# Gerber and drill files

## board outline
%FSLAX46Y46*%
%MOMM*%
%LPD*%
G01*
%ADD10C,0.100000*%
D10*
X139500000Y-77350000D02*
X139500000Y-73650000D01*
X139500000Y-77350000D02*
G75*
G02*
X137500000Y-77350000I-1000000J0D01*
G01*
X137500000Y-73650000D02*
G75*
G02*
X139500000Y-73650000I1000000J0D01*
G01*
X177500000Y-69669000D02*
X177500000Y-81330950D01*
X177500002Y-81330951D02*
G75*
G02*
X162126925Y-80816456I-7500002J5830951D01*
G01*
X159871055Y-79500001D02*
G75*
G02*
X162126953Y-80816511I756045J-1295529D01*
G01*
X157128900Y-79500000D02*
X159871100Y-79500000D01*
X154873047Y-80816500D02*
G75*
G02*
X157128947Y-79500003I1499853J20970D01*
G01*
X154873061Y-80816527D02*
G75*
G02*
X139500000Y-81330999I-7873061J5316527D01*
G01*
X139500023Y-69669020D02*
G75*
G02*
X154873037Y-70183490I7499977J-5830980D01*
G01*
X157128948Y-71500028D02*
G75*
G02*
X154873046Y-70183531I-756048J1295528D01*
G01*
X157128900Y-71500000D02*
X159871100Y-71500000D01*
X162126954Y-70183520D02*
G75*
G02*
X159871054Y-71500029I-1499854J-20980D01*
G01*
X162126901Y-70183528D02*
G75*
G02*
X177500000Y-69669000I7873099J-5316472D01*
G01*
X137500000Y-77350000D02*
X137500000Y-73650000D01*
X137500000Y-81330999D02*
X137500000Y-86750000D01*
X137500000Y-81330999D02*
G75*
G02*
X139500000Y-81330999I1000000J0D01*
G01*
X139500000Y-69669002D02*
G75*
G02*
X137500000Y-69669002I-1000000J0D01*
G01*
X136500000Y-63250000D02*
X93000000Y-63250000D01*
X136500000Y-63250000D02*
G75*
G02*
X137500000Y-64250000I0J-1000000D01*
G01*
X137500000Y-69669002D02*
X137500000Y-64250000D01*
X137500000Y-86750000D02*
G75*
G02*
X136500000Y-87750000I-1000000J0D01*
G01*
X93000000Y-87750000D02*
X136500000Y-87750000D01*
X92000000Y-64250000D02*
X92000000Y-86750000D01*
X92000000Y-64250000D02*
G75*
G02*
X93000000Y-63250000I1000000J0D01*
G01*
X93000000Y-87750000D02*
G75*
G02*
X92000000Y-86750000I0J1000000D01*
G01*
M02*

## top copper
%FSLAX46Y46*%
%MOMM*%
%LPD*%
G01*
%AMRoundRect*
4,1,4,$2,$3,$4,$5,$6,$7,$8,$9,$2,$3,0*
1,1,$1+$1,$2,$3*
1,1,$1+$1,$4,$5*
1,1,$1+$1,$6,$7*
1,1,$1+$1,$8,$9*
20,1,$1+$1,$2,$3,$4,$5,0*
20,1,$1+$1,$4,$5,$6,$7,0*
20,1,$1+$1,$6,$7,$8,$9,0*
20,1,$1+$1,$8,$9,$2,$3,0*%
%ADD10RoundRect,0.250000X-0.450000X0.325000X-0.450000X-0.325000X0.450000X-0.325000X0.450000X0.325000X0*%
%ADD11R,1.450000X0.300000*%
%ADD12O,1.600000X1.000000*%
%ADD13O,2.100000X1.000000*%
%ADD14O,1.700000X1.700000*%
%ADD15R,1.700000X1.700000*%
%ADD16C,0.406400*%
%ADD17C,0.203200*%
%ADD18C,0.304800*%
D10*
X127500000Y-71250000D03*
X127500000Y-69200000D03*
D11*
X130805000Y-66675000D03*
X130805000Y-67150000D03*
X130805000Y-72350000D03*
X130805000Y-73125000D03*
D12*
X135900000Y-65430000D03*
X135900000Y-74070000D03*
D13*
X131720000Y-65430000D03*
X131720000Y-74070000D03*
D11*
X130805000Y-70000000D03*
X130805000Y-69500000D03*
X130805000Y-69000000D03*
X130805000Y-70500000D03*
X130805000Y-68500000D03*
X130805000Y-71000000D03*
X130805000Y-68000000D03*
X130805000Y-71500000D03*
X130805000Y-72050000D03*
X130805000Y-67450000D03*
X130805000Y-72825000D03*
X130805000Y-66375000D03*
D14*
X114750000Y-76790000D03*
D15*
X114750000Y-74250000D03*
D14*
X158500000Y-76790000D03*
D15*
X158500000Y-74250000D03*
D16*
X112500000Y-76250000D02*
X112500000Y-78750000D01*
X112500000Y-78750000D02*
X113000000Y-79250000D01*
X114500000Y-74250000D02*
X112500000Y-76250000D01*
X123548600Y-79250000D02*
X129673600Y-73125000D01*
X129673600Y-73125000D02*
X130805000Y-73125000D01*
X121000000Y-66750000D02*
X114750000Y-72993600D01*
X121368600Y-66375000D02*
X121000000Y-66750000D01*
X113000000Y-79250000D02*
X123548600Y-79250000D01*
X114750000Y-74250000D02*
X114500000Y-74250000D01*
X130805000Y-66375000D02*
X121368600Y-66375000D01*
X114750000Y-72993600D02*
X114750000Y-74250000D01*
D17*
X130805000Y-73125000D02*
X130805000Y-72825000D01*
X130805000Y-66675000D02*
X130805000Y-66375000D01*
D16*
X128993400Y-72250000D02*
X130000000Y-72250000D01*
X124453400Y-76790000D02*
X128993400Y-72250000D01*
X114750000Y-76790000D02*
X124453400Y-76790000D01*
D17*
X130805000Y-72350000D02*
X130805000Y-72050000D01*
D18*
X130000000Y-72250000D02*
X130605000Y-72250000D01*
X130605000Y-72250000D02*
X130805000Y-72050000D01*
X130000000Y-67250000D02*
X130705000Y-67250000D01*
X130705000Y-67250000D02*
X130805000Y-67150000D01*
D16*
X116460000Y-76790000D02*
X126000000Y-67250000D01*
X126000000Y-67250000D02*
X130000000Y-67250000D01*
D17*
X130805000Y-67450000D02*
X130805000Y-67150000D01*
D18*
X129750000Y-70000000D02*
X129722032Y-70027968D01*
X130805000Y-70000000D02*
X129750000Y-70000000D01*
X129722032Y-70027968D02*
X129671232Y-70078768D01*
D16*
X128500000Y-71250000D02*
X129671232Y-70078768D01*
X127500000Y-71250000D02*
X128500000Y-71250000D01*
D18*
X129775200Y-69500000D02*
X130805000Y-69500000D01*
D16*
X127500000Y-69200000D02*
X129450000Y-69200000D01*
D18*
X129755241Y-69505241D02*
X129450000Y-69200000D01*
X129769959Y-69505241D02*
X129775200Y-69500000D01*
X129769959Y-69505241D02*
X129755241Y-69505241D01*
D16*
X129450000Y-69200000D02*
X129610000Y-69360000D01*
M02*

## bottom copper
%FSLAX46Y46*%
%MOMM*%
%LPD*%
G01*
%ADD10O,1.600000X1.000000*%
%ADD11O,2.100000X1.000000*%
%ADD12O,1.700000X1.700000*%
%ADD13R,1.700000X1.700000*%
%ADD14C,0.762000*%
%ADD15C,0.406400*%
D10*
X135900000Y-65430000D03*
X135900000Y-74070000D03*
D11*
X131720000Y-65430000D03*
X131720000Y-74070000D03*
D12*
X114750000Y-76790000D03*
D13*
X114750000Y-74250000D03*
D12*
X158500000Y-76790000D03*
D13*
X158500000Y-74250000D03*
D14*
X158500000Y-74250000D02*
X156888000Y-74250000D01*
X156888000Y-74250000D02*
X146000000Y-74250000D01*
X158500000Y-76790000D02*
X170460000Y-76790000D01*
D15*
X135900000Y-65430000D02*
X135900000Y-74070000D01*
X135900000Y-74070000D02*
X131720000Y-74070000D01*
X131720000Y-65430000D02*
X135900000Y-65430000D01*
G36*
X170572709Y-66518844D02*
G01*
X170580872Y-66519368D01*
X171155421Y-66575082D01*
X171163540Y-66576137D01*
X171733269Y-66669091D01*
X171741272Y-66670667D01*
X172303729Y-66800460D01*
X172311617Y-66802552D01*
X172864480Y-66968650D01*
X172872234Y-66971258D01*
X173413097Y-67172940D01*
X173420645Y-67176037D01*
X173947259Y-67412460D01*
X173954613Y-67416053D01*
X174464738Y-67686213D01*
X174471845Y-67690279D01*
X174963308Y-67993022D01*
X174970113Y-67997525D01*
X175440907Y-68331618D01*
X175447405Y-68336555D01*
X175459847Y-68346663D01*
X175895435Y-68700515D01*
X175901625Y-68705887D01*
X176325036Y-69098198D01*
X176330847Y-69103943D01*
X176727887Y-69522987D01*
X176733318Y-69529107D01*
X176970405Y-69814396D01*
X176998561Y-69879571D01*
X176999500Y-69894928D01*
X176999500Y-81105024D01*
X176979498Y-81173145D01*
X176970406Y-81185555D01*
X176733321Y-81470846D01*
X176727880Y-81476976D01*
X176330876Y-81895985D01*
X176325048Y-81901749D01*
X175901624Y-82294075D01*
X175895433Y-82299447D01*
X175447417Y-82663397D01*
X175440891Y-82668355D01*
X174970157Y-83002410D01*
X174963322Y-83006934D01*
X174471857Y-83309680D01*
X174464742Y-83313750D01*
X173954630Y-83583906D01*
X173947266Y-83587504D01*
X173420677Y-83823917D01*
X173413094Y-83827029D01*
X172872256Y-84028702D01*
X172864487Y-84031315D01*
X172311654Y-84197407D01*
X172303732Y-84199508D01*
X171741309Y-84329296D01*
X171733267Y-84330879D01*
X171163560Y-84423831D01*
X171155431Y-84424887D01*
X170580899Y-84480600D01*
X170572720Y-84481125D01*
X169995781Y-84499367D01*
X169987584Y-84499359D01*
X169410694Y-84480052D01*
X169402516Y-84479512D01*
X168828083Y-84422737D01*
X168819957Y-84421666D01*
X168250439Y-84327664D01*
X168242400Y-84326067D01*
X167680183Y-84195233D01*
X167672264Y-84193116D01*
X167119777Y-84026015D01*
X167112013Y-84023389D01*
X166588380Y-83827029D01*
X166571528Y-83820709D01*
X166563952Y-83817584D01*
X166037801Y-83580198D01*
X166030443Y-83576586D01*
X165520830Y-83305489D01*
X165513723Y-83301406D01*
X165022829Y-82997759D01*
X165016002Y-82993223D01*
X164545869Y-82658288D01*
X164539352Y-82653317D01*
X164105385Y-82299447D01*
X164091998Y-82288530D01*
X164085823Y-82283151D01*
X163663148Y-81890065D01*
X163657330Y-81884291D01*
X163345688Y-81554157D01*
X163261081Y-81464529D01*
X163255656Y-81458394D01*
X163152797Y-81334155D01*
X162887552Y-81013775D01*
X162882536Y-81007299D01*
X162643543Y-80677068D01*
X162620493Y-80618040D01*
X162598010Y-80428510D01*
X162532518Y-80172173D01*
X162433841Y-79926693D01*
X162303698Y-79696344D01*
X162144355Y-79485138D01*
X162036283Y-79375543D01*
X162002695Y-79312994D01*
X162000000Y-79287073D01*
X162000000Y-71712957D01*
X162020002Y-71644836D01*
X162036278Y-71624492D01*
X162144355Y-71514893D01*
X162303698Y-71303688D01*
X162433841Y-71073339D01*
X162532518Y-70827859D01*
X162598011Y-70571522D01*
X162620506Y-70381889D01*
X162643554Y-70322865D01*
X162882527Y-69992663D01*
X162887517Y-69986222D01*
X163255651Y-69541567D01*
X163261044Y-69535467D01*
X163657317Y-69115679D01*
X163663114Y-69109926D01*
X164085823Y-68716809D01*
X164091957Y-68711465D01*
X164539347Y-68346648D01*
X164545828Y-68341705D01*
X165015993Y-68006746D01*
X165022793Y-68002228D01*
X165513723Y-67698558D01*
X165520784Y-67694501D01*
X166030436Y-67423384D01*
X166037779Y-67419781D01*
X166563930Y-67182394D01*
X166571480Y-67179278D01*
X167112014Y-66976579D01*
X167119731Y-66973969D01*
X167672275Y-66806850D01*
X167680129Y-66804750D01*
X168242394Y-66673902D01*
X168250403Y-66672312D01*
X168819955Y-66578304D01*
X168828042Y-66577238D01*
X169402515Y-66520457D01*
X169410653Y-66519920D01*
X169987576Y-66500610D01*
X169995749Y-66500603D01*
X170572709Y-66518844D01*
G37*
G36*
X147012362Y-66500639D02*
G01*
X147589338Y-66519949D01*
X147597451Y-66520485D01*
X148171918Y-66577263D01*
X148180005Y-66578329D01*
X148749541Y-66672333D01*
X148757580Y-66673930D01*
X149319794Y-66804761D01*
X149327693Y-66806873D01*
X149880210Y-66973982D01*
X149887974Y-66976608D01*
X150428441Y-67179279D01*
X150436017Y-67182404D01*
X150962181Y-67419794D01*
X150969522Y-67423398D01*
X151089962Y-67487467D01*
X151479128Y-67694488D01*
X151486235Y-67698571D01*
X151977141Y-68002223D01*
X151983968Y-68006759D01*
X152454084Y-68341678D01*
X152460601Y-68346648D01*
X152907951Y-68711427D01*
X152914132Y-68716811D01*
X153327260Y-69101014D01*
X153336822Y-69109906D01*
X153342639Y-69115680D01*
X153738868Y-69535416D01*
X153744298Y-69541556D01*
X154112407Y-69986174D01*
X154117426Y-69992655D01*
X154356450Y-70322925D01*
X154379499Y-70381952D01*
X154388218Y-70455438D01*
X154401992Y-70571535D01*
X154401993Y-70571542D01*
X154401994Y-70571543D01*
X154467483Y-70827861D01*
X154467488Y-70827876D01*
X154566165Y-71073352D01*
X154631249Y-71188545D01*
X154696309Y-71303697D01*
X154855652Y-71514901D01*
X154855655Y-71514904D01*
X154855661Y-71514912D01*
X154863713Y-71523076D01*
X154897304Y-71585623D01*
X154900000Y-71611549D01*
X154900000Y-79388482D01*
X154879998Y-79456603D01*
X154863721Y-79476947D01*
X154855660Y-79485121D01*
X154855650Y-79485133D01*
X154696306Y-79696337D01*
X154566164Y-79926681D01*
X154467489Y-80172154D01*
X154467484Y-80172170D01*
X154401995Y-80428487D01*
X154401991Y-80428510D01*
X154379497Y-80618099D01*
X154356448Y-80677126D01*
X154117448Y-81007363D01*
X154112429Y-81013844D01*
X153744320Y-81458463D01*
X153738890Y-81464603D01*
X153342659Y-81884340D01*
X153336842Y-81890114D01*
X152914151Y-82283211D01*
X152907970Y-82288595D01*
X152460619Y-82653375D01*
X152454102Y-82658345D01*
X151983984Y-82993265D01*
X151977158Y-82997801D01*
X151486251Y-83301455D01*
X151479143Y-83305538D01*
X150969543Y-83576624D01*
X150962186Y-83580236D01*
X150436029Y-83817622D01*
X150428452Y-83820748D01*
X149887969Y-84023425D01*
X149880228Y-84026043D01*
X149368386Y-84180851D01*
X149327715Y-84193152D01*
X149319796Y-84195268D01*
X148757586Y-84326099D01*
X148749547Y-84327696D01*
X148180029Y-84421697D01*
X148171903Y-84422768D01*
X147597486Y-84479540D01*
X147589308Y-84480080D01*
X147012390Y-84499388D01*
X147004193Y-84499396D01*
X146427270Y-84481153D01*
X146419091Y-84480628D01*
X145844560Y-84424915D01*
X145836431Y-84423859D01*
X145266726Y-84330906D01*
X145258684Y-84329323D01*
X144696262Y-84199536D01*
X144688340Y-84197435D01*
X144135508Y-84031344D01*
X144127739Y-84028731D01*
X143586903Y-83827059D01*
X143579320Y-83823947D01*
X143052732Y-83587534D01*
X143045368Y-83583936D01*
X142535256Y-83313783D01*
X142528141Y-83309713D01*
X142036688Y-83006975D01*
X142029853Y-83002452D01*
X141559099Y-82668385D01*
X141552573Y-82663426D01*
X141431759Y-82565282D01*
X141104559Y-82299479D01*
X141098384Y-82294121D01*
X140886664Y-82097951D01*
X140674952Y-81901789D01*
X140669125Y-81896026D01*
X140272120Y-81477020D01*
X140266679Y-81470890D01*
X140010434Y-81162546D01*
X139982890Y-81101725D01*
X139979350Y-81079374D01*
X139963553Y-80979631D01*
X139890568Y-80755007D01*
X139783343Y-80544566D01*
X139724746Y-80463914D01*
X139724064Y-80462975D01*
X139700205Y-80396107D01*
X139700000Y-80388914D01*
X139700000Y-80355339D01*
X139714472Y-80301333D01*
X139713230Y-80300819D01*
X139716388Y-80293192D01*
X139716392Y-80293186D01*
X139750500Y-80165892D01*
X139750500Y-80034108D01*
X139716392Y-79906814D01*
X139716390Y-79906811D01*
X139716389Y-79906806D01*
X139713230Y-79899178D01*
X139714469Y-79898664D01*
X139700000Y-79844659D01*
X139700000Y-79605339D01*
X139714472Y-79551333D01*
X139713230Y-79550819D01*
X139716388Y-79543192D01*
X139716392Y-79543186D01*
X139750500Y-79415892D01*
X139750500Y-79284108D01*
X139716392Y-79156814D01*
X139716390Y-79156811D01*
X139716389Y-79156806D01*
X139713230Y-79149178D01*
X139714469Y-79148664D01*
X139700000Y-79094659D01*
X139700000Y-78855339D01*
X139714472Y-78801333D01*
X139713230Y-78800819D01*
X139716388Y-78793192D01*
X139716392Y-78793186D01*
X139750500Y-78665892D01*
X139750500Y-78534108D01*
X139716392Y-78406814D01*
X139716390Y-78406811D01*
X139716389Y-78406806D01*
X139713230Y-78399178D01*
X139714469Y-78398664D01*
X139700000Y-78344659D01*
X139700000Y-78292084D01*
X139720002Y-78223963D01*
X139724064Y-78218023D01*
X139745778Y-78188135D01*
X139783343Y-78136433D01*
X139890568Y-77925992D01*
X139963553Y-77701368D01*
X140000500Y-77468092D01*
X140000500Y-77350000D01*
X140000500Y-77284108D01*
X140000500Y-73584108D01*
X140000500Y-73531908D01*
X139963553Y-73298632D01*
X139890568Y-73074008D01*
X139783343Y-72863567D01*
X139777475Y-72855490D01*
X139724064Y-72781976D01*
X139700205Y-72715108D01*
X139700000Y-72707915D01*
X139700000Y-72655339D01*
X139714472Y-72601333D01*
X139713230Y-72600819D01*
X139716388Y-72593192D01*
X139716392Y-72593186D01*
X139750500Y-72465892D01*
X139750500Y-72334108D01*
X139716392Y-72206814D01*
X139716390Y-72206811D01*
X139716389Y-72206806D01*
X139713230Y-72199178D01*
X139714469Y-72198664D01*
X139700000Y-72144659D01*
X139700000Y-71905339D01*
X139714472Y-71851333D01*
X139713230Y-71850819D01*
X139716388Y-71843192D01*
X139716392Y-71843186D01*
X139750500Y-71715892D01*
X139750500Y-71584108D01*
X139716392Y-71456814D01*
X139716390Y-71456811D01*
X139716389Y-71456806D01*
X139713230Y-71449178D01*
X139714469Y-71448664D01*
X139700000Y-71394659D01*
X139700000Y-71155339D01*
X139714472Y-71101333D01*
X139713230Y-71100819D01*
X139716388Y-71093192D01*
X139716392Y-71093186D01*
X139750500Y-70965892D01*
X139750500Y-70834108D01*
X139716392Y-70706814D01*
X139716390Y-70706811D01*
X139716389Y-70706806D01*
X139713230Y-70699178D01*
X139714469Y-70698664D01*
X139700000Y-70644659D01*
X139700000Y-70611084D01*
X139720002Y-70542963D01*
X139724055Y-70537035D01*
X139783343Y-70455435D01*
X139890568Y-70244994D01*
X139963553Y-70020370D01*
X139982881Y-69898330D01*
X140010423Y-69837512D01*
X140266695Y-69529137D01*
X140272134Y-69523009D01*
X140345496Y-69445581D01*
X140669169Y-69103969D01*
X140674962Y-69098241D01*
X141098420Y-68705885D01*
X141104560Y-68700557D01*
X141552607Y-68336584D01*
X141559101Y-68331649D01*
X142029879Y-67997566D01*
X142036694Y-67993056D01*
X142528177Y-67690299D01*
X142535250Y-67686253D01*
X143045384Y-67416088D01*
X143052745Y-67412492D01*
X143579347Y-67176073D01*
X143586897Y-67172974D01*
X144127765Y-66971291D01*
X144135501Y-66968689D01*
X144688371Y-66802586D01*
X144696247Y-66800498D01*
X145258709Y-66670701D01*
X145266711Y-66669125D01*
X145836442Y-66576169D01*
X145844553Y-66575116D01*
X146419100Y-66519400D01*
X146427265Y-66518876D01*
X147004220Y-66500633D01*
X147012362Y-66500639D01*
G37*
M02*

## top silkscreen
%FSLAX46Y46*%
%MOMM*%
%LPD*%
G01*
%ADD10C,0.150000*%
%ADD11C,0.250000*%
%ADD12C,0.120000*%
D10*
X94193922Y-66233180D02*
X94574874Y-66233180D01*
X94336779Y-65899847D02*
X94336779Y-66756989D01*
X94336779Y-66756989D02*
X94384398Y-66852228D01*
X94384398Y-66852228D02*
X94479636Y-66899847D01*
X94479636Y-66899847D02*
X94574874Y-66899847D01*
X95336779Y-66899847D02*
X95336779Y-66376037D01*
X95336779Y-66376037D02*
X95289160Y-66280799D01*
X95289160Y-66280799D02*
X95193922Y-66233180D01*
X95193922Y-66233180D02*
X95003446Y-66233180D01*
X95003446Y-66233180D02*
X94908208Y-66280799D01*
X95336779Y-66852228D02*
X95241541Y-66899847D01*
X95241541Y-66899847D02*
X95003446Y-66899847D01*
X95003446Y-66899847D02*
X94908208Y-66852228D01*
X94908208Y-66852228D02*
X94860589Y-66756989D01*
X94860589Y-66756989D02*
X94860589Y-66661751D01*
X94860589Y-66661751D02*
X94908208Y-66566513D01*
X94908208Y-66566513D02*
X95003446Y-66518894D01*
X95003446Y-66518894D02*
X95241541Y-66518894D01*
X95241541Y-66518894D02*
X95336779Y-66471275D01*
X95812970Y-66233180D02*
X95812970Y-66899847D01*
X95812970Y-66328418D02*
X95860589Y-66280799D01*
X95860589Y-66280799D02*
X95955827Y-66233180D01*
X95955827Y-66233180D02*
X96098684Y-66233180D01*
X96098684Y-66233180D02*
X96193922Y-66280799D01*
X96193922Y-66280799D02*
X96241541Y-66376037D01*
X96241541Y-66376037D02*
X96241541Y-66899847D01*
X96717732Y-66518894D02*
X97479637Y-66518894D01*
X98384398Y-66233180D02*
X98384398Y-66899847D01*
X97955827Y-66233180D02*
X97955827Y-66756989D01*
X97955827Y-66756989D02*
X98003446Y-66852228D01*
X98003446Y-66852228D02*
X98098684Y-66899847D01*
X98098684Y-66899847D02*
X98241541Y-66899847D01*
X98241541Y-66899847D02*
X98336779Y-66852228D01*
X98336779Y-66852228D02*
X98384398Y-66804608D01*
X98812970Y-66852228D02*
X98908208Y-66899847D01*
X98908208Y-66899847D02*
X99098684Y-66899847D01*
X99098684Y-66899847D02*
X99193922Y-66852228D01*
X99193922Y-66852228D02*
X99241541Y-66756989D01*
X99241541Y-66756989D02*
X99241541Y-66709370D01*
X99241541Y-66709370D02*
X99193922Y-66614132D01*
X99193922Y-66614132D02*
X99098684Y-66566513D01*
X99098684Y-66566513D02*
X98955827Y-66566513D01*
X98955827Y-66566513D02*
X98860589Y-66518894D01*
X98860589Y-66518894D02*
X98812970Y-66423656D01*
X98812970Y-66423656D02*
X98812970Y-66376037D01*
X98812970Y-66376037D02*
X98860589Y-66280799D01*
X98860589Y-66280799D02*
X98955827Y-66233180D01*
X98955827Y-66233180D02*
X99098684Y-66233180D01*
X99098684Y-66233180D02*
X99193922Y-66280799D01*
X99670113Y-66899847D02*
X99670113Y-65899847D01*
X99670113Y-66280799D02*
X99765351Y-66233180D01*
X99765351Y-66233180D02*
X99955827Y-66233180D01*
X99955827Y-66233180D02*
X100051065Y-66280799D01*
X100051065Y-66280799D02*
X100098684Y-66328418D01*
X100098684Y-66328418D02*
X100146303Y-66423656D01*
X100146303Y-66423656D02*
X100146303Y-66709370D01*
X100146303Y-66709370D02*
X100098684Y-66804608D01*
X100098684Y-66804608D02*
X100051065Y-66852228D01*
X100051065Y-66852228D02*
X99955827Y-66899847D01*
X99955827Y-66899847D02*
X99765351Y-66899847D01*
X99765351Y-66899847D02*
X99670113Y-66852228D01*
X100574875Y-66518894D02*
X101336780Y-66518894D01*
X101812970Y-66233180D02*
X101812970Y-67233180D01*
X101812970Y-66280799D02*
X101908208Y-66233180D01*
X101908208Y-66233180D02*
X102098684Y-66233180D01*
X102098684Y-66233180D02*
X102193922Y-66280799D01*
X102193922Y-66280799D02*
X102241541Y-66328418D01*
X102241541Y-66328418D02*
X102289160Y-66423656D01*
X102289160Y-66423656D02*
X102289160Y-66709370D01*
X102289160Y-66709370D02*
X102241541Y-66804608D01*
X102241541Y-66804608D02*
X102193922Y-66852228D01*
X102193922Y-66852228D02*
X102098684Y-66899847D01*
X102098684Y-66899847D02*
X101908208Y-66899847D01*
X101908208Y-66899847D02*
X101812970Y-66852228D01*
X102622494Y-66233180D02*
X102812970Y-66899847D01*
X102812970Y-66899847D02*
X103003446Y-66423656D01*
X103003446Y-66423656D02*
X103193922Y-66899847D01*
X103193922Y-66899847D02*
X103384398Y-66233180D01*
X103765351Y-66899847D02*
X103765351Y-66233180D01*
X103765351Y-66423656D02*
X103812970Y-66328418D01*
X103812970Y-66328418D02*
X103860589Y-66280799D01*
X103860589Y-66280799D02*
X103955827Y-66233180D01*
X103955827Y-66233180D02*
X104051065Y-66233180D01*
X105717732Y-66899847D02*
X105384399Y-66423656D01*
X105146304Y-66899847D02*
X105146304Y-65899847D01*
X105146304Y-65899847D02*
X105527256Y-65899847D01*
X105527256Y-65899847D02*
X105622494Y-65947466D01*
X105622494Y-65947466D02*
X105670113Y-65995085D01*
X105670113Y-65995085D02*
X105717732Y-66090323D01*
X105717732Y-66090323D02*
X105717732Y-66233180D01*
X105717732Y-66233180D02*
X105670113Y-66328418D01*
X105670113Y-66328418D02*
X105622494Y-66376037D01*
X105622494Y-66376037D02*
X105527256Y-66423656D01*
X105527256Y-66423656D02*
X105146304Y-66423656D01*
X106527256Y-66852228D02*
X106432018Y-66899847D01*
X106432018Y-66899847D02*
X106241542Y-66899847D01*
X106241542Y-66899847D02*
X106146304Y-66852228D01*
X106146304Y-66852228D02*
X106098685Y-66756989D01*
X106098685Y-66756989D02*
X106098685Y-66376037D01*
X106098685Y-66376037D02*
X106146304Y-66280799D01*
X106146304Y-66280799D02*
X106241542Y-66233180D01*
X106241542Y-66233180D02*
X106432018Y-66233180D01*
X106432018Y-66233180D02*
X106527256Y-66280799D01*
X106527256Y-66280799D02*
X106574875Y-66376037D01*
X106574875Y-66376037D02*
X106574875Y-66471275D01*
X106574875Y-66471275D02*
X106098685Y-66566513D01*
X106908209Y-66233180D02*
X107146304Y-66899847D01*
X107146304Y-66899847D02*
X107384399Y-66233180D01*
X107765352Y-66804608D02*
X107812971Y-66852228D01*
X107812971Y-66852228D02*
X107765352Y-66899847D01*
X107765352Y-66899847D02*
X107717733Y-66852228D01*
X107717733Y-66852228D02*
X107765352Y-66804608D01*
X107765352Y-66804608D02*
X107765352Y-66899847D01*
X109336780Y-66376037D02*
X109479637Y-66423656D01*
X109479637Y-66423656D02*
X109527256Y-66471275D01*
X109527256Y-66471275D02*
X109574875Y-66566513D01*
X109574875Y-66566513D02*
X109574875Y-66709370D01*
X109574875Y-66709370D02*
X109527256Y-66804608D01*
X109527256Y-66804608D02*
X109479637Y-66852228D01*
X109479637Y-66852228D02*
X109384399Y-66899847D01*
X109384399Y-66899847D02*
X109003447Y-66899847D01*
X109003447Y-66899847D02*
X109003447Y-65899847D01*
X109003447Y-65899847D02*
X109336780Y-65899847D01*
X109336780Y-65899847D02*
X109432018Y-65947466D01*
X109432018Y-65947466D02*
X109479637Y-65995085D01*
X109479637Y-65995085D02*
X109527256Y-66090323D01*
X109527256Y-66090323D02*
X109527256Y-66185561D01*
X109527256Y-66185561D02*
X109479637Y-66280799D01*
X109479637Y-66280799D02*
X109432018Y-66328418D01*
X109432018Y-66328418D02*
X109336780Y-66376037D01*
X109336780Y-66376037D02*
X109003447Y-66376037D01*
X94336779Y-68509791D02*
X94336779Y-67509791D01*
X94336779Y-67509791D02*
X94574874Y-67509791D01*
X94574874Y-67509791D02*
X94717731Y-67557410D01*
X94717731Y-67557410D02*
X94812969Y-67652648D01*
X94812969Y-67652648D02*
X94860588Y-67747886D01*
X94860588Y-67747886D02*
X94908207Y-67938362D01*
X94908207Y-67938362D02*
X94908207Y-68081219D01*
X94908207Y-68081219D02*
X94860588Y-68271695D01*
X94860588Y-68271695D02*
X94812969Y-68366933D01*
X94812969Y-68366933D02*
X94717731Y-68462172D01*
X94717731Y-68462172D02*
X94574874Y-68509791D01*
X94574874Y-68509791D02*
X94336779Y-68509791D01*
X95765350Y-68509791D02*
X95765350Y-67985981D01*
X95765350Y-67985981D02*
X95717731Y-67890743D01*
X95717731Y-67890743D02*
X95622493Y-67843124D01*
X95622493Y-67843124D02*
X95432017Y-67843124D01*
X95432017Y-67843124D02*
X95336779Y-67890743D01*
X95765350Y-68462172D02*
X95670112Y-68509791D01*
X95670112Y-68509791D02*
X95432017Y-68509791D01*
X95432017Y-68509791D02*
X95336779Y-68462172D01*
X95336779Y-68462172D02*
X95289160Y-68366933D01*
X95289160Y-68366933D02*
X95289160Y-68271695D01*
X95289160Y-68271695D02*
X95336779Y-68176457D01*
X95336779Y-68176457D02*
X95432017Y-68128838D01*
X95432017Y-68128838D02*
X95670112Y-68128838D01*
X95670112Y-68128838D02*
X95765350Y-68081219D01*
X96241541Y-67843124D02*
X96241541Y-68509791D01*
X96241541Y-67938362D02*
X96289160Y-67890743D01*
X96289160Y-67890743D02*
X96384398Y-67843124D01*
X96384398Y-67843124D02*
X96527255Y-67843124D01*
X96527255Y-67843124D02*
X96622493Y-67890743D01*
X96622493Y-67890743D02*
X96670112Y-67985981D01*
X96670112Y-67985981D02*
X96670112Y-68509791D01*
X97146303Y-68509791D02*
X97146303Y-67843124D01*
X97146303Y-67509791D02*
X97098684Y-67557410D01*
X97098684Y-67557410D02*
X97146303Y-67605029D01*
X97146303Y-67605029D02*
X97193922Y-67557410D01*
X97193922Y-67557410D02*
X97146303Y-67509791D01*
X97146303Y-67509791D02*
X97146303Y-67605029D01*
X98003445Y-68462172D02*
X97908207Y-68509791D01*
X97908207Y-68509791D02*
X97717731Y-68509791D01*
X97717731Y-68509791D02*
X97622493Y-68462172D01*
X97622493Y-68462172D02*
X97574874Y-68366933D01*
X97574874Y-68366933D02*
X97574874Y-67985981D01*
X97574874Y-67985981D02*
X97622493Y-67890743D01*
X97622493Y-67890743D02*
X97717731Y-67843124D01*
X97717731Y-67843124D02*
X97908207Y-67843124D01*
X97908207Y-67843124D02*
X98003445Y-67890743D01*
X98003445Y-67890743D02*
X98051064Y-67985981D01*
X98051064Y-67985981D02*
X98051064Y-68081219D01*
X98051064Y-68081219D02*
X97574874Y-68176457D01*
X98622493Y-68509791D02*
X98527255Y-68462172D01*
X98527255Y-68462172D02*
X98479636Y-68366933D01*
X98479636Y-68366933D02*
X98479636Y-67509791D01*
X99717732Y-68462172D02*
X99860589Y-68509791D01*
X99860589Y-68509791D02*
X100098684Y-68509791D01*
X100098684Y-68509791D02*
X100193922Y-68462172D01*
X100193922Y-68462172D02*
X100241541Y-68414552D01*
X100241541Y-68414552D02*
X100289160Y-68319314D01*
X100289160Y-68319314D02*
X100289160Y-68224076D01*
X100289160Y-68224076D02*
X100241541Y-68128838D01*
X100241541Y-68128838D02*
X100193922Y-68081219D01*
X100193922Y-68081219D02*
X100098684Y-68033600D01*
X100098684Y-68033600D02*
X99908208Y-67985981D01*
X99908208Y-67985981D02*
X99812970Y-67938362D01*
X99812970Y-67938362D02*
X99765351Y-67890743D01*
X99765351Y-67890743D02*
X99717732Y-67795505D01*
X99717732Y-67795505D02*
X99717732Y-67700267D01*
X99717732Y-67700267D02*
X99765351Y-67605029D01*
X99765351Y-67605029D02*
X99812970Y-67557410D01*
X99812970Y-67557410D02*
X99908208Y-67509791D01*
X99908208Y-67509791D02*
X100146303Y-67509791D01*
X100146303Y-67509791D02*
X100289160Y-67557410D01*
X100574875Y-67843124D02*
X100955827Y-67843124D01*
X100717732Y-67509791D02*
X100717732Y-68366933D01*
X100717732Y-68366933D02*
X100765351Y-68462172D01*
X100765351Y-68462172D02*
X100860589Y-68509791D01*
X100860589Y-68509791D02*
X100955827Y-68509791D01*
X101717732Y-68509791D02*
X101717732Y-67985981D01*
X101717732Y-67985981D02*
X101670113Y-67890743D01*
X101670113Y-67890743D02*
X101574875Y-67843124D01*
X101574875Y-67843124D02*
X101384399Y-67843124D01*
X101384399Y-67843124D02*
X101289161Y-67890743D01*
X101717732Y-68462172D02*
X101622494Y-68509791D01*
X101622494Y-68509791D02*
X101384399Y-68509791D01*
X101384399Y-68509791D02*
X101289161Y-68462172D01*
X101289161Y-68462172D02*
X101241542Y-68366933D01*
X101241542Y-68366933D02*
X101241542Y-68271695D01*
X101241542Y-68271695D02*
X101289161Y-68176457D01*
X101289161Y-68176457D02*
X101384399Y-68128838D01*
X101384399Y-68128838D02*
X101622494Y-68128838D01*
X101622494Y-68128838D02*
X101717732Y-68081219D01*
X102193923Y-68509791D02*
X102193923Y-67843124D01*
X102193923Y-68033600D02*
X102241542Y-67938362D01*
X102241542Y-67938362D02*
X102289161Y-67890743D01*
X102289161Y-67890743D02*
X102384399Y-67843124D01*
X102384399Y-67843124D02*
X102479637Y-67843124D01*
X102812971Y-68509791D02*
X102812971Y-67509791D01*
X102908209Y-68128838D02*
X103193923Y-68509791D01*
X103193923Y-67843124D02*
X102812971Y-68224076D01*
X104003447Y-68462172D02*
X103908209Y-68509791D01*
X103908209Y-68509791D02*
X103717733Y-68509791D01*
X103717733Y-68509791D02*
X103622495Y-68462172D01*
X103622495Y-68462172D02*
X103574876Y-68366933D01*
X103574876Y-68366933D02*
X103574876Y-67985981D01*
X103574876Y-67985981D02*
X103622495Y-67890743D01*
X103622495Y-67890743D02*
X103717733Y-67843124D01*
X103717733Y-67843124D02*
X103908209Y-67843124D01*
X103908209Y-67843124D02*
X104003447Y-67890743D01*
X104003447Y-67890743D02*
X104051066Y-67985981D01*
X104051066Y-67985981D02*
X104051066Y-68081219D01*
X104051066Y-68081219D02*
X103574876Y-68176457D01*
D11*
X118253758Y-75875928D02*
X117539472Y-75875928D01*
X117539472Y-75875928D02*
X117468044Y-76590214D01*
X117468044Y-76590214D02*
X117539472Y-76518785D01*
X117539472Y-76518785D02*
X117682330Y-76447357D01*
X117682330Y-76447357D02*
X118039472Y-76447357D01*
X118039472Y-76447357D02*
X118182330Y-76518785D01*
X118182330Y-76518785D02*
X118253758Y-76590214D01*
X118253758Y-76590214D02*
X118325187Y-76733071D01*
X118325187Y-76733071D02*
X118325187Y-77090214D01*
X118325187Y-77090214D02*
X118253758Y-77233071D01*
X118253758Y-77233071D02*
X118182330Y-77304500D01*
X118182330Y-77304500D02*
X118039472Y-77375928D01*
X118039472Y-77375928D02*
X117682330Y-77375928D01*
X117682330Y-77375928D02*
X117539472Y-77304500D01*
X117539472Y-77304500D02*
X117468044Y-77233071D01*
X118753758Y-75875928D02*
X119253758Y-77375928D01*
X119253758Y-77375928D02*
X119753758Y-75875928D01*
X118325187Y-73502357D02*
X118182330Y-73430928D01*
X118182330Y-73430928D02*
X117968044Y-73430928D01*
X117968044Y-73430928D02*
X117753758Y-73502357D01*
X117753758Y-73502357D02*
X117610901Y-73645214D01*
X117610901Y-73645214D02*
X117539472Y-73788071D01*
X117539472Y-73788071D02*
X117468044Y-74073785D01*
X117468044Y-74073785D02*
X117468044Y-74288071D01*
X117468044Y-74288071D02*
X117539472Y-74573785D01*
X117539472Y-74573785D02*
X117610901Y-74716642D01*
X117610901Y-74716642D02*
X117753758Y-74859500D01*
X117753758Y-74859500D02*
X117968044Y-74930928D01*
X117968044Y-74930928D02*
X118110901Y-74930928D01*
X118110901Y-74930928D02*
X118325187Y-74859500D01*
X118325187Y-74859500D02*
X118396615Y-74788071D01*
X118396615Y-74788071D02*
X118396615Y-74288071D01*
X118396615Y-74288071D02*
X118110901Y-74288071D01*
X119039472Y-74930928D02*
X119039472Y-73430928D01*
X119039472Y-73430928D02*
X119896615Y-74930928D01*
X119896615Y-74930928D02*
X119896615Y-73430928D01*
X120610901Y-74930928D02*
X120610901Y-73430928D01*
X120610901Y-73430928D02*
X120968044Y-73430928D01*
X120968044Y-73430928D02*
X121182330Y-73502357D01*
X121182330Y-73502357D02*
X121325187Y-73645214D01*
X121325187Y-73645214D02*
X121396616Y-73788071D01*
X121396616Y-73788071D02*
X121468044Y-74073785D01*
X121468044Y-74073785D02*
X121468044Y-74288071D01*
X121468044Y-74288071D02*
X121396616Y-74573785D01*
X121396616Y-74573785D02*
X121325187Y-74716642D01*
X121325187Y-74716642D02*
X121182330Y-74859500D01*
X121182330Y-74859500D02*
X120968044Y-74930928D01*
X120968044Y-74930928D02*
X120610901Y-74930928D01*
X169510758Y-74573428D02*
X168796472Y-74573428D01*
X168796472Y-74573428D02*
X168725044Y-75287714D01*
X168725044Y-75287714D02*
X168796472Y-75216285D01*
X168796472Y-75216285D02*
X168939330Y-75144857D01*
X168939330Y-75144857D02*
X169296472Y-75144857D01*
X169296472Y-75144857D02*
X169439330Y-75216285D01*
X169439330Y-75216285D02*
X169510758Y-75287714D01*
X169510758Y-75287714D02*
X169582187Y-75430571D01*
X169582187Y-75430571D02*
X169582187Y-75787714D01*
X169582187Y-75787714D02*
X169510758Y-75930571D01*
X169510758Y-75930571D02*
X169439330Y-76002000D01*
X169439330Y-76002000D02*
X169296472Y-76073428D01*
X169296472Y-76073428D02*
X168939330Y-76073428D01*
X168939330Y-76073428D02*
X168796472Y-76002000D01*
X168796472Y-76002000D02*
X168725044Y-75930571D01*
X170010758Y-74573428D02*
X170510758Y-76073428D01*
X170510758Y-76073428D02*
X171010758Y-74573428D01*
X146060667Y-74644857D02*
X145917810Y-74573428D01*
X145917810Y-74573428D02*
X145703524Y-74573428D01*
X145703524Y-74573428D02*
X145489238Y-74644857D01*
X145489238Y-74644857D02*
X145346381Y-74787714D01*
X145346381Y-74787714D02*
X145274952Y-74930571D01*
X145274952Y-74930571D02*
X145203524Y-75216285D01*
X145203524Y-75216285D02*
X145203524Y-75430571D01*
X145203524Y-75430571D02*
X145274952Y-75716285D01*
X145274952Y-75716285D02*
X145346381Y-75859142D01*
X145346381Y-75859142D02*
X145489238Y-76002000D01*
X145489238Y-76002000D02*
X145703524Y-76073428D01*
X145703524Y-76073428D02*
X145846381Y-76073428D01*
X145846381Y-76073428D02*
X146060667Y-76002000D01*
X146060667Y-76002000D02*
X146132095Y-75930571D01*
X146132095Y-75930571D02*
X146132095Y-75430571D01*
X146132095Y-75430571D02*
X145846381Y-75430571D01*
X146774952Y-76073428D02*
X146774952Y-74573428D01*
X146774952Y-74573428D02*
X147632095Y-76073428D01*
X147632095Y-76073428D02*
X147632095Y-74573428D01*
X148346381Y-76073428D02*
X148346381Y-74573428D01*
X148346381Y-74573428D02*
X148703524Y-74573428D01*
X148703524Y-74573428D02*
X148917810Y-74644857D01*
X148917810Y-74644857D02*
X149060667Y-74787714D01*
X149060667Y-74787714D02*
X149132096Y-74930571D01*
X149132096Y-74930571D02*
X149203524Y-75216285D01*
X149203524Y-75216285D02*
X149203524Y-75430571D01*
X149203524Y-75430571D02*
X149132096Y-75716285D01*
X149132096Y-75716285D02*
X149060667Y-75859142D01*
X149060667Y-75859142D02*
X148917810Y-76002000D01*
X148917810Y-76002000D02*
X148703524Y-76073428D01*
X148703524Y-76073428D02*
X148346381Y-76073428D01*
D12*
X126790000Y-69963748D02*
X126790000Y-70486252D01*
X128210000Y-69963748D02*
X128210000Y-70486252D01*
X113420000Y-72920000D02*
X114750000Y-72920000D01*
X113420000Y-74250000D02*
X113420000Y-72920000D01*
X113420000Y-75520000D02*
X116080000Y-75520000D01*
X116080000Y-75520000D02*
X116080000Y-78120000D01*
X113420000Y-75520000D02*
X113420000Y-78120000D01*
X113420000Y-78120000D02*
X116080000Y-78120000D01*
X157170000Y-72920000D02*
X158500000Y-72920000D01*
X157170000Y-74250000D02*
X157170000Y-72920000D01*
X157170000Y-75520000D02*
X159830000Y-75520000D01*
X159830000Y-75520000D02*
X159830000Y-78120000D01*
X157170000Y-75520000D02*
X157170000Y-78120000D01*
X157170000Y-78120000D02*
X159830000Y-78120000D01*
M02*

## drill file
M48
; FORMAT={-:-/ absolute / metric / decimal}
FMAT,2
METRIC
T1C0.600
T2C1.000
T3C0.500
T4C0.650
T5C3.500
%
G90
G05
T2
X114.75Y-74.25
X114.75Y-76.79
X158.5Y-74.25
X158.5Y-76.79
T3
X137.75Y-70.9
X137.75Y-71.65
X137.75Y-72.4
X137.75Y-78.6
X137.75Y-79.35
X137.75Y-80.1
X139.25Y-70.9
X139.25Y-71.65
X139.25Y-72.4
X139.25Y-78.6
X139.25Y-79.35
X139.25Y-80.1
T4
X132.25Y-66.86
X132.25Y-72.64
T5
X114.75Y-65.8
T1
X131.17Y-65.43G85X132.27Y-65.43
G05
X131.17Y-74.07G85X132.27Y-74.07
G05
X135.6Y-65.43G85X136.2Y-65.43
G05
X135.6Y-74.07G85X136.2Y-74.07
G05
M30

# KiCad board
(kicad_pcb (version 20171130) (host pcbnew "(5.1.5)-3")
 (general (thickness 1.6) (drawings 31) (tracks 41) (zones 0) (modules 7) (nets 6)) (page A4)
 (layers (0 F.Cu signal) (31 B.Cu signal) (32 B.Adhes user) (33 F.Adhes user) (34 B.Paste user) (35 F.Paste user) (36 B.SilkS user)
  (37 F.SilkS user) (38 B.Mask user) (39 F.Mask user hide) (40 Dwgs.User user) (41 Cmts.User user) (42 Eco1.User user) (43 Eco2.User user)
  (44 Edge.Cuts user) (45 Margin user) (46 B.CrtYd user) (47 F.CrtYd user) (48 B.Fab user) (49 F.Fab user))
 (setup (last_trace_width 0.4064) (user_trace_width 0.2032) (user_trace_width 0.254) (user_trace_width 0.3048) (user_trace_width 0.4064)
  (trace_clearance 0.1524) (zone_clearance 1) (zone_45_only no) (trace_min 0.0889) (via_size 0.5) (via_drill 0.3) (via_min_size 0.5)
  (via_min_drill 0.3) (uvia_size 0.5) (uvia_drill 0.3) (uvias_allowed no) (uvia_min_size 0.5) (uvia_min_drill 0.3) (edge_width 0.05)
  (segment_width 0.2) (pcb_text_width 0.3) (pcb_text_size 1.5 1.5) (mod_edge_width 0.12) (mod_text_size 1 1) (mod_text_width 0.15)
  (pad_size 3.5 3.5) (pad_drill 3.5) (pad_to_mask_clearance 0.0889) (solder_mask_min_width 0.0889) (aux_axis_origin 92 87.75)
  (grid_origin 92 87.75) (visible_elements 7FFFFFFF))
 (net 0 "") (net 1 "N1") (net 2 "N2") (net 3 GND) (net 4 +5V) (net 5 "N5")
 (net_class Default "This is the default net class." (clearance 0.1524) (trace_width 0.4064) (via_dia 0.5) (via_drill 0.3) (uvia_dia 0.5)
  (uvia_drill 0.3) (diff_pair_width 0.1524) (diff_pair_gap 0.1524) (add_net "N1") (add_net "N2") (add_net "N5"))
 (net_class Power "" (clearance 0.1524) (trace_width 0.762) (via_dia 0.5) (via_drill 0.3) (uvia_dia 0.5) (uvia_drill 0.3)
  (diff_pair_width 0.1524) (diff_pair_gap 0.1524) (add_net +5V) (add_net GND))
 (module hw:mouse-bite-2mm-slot (layer F.Cu) (at 138.5 79.35 90)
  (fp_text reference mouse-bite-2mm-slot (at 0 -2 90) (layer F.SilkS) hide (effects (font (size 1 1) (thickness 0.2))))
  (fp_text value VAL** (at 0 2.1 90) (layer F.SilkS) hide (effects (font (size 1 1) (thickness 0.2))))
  (pad "" np_thru_hole circle (at 0 -0.75 90) (size 0.5 0.5) (drill 0.5) (layers *.Cu *.Mask))
  (pad "" np_thru_hole circle (at 0 0.75 90) (size 0.5 0.5) (drill 0.5) (layers *.Cu *.Mask))
  (pad "" np_thru_hole circle (at 0.75 -0.75 90) (size 0.5 0.5) (drill 0.5) (layers *.Cu *.Mask))
  (pad "" np_thru_hole circle (at -0.75 -0.75 90) (size 0.5 0.5) (drill 0.5) (layers *.Cu *.Mask))
  (pad "" np_thru_hole circle (at -0.75 0.75 90) (size 0.5 0.5) (drill 0.5) (layers *.Cu *.Mask))
  (pad "" np_thru_hole circle (at 0.75 0.75 90) (size 0.5 0.5) (drill 0.5) (layers *.Cu *.Mask)))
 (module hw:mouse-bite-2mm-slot (layer F.Cu) (at 138.5 71.65 90)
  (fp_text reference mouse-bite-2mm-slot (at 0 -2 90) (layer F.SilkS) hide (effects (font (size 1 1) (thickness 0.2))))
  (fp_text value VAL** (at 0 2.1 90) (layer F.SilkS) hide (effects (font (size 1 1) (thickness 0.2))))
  (pad "" np_thru_hole circle (at 0 -0.75 90) (size 0.5 0.5) (drill 0.5) (layers *.Cu *.Mask))
  (pad "" np_thru_hole circle (at 0 0.75 90) (size 0.5 0.5) (drill 0.5) (layers *.Cu *.Mask))
  (pad "" np_thru_hole circle (at 0.75 -0.75 90) (size 0.5 0.5) (drill 0.5) (layers *.Cu *.Mask))
  (pad "" np_thru_hole circle (at -0.75 -0.75 90) (size 0.5 0.5) (drill 0.5) (layers *.Cu *.Mask))
  (pad "" np_thru_hole circle (at -0.75 0.75 90) (size 0.5 0.5) (drill 0.5) (layers *.Cu *.Mask))
  (pad "" np_thru_hole circle (at 0.75 0.75 90) (size 0.5 0.5) (drill 0.5) (layers *.Cu *.Mask)))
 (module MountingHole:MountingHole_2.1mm (layer F.Cu) (at 114.75 65.8)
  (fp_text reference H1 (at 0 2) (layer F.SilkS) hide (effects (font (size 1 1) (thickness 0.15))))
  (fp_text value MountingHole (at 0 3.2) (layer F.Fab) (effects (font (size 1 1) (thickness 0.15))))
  (pad "" np_thru_hole circle (at 0 0) (size 3.5 3.5) (drill 3.5) (layers *.Cu *.Mask)))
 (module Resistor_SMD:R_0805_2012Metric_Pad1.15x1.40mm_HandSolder (layer F.Cu) (at 127.5 70.225 270)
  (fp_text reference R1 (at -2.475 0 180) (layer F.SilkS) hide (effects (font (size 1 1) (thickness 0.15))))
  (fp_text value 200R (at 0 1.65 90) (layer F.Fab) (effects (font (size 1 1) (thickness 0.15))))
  (fp_line (start -0.261252 0.71) (end 0.261252 0.71) (layer F.SilkS) (width 0.12))
  (fp_line (start -0.261252 -0.71) (end 0.261252 -0.71) (layer F.SilkS) (width 0.12))
  (pad 2 smd roundrect (at 1.025 0 270) (size 1.15 1.4) (layers F.Cu F.Paste F.Mask) (roundrect_rratio 0.217391) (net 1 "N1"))
  (pad 1 smd roundrect (at -1.025 0 270) (size 1.15 1.4) (layers F.Cu F.Paste F.Mask) (roundrect_rratio 0.217391) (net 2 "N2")))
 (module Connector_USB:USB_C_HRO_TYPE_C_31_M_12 (layer F.Cu) (at 138.5 69.75 90)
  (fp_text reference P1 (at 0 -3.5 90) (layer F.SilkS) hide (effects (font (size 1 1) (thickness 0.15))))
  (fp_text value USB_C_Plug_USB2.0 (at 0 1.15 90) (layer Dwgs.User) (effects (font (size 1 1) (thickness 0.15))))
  (pad B1 smd rect (at 3.075 -7.695 90) (size 0.3 1.45) (layers F.Cu F.Paste F.Mask) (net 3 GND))
  (pad A9 smd rect (at 2.6 -7.695 90) (size 0.3 1.45) (layers F.Cu F.Paste F.Mask) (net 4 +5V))
  (pad A4 smd rect (at -2.6 -7.695 90) (size 0.3 1.45) (layers F.Cu F.Paste F.Mask) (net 4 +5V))
  (pad A1 smd rect (at -3.375 -7.695 90) (size 0.3 1.45) (layers F.Cu F.Paste F.Mask) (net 3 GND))
  (pad S1 thru_hole oval (at 4.32 -2.6 90) (size 1 1.6) (drill oval 0.6 1.2) (layers *.Cu *.Mask) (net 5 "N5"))
  (pad S1 thru_hole oval (at -4.32 -2.6 90) (size 1 1.6) (drill oval 0.6 1.2) (layers *.Cu *.Mask) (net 5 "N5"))
  (pad S1 thru_hole oval (at 4.32 -6.78 90) (size 1 2.1) (drill oval 0.6 1.7) (layers *.Cu *.Mask) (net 5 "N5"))
  (pad S1 thru_hole oval (at -4.32 -6.78 90) (size 1 2.1) (drill oval 0.6 1.7) (layers *.Cu *.Mask) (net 5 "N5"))
  (pad "" np_thru_hole circle (at -2.89 -6.25 90) (size 0.65 0.65) (drill 0.65) (layers *.Cu *.Mask))
  (pad "" np_thru_hole circle (at 2.89 -6.25 90) (size 0.65 0.65) (drill 0.65) (layers *.Cu *.Mask))
  (pad A6 smd rect (at -0.25 -7.695 90) (size 0.3 1.45) (layers F.Cu F.Paste F.Mask) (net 1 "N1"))
  (pad A7 smd rect (at 0.25 -7.695 90) (size 0.3 1.45) (layers F.Cu F.Paste F.Mask) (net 2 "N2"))
  (pad B6 smd rect (at 0.75 -7.695 90) (size 0.3 1.45) (layers F.Cu F.Paste F.Mask))
  (pad B7 smd rect (at -0.75 -7.695 90) (size 0.3 1.45) (layers F.Cu F.Paste F.Mask))
  (pad A8 smd rect (at 1.25 -7.695 90) (size 0.3 1.45) (layers F.Cu F.Paste F.Mask))
  (pad A5 smd rect (at -1.25 -7.695 90) (size 0.3 1.45) (layers F.Cu F.Paste F.Mask))
  (pad B5 smd rect (at 1.75 -7.695 90) (size 0.3 1.45) (layers F.Cu F.Paste F.Mask))
  (pad B8 smd rect (at -1.75 -7.695 90) (size 0.3 1.45) (layers F.Cu F.Paste F.Mask))
  (pad B9 smd rect (at -2.3 -7.695 90) (size 0.3 1.45) (layers F.Cu F.Paste F.Mask) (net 4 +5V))
  (pad B4 smd rect (at 2.3 -7.695 90) (size 0.3 1.45) (layers F.Cu F.Paste F.Mask) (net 4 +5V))
  (pad B12 smd rect (at -3.075 -7.695 90) (size 0.3 1.45) (layers F.Cu F.Paste F.Mask) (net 3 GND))
  (pad A12 smd rect (at 3.375 -7.695 90) (size 0.3 1.45) (layers F.Cu F.Paste F.Mask) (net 3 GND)))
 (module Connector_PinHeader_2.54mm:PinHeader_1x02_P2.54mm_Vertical (layer F.Cu) (at 114.75 74.25)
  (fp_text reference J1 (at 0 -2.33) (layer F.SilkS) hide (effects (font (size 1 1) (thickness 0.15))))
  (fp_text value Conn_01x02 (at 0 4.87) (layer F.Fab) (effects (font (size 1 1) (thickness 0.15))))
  (fp_line (start -1.33 -1.33) (end 0 -1.33) (layer F.SilkS) (width 0.12))
  (fp_line (start -1.33 0) (end -1.33 -1.33) (layer F.SilkS) (width 0.12))
  (fp_line (start -1.33 1.27) (end 1.33 1.27) (layer F.SilkS) (width 0.12))
  (fp_line (start 1.33 1.27) (end 1.33 3.87) (layer F.SilkS) (width 0.12))
  (fp_line (start -1.33 1.27) (end -1.33 3.87) (layer F.SilkS) (width 0.12))
  (fp_line (start -1.33 3.87) (end 1.33 3.87) (layer F.SilkS) (width 0.12))
  (pad 2 thru_hole oval (at 0 2.54) (size 1.7 1.7) (drill 1) (layers *.Cu *.Mask) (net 4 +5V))
  (pad 1 thru_hole rect (at 0 0) (size 1.7 1.7) (drill 1) (layers *.Cu *.Mask) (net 3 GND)))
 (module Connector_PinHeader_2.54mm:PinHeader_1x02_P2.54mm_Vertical (layer F.Cu) (at 158.5 74.25)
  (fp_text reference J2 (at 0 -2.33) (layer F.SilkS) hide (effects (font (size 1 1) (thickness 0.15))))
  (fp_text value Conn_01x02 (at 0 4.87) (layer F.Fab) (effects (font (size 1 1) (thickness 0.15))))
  (fp_line (start -1.33 -1.33) (end 0 -1.33) (layer F.SilkS) (width 0.12))
  (fp_line (start -1.33 0) (end -1.33 -1.33) (layer F.SilkS) (width 0.12))
  (fp_line (start -1.33 1.27) (end 1.33 1.27) (layer F.SilkS) (width 0.12))
  (fp_line (start 1.33 1.27) (end 1.33 3.87) (layer F.SilkS) (width 0.12))
  (fp_line (start -1.33 1.27) (end -1.33 3.87) (layer F.SilkS) (width 0.12))
  (fp_line (start -1.33 3.87) (end 1.33 3.87) (layer F.SilkS) (width 0.12))
  (pad 2 thru_hole oval (at 0 2.54) (size 1.7 1.7) (drill 1) (layers *.Cu *.Mask) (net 4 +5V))
  (pad 1 thru_hole rect (at 0 0) (size 1.7 1.7) (drill 1) (layers *.Cu *.Mask) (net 3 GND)))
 (gr_line (start 139.5 77.35) (end 139.5 73.65) (layer Edge.Cuts) (width 0.1))
 (gr_arc (start 138.5 77.35) (end 137.5 77.35) (angle -180) (layer Edge.Cuts) (width 0.1))
 (gr_arc (start 138.5 73.65) (end 139.5 73.65) (angle -180) (layer Edge.Cuts) (width 0.1))
 (gr_line (start 177.5 69.669) (end 177.5 81.33095) (layer Edge.Cuts) (width 0.1))
 (gr_arc (start 170 75.5) (end 162.126925 80.816456) (angle -108.1063631) (layer Edge.Cuts) (width 0.1))
 (gr_arc (start 160.6271 80.79553) (end 162.126953 80.816511) (angle -121.06842) (layer Edge.Cuts) (width 0.1))
 (gr_line (start 157.1289 79.5) (end 159.8711 79.5) (layer Edge.Cuts) (width 0.1))
 (gr_arc (start 156.3729 80.79553) (end 157.128947 79.500003) (angle -121.0681) (layer Edge.Cuts) (width 0.1))
 (gr_arc (start 147 75.5) (end 139.5 81.330999) (angle -108.1057277) (layer Edge.Cuts) (width 0.1))
 (gr_arc (start 147 75.5) (end 154.873037 70.18349) (angle -108.1057364) (layer Edge.Cuts) (width 0.1))
 (gr_arc (start 156.3729 70.2045) (end 154.873046 70.183531) (angle -121.0681) (layer Edge.Cuts) (width 0.1))
 (gr_line (start 157.1289 71.5) (end 159.8711 71.5) (layer Edge.Cuts) (width 0.1))
 (gr_arc (start 160.6271 70.2045) (end 159.871054 71.500029) (angle -121.06842) (layer Edge.Cuts) (width 0.1))
 (gr_arc (start 170 75.5) (end 177.5 69.669) (angle -108.1061261) (layer Edge.Cuts) (width 0.1))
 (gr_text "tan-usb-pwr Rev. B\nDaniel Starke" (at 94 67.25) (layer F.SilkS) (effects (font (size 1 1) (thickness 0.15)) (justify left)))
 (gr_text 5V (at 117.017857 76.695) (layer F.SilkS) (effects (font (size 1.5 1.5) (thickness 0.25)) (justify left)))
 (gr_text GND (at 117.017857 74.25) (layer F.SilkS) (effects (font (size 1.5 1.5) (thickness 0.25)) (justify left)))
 (gr_line (start 137.5 77.35) (end 137.5 73.65) (layer Edge.Cuts) (width 0.1))
 (gr_line (start 137.5 81.330999) (end 137.5 86.75) (layer Edge.Cuts) (width 0.1))
 (gr_arc (start 138.5 81.330999) (end 139.5 81.330999) (angle -180) (layer Edge.Cuts) (width 0.1))
 (gr_arc (start 138.5 69.669002) (end 137.5 69.669002) (angle -180) (layer Edge.Cuts) (width 0.1))
 (gr_line (start 136.5 63.25) (end 93 63.25) (layer Edge.Cuts) (width 0.1))
 (gr_arc (start 136.5 64.25) (end 137.5 64.25) (angle -90) (layer Edge.Cuts) (width 0.1))
 (gr_line (start 137.5 69.669002) (end 137.5 64.25) (layer Edge.Cuts) (width 0.1))
 (gr_arc (start 136.5 86.75) (end 136.5 87.75) (angle -90) (layer Edge.Cuts) (width 0.1))
 (gr_line (start 93 87.75) (end 136.5 87.75) (layer Edge.Cuts) (width 0.1))
 (gr_line (start 92 64.25) (end 92 86.75) (layer Edge.Cuts) (width 0.1))
 (gr_arc (start 93 64.25) (end 93 63.25) (angle -90) (layer Edge.Cuts) (width 0.1))
 (gr_arc (start 93 86.75) (end 92 86.75) (angle -90) (layer Edge.Cuts) (width 0.1))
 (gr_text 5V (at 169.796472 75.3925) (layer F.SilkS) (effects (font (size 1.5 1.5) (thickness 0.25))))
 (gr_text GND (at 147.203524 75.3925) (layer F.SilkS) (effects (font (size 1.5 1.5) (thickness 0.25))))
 (segment (start 158.5 74.25) (end 156.888 74.25) (width 0.762) (layer B.Cu) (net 3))
 (segment (start 156.888 74.25) (end 146 74.25) (width 0.762) (layer B.Cu) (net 3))
 (segment (start 112.5 76.25) (end 112.5 78.75) (width 0.4064) (layer F.Cu) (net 3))
 (segment (start 112.5 78.75) (end 113 79.25) (width 0.4064) (layer F.Cu) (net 3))
 (segment (start 114.5 74.25) (end 112.5 76.25) (width 0.4064) (layer F.Cu) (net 3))
 (segment (start 123.5486 79.25) (end 129.6736 73.125) (width 0.4064) (layer F.Cu) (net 3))
 (segment (start 129.6736 73.125) (end 130.805 73.125) (width 0.4064) (layer F.Cu) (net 3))
 (segment (start 121 66.75) (end 114.75 72.9936) (width 0.4064) (layer F.Cu) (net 3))
 (segment (start 121.3686 66.375) (end 121 66.75) (width 0.4064) (layer F.Cu) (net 3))
 (segment (start 113 79.25) (end 123.5486 79.25) (width 0.4064) (layer F.Cu) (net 3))
 (segment (start 114.75 74.25) (end 114.5 74.25) (width 0.4064) (layer F.Cu) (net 3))
 (segment (start 130.805 66.375) (end 121.3686 66.375) (width 0.4064) (layer F.Cu) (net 3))
 (segment (start 114.75 72.9936) (end 114.75 74.25) (width 0.4064) (layer F.Cu) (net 3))
 (segment (start 130.805 73.125) (end 130.805 72.825) (width 0.2032) (layer F.Cu) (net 3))
 (segment (start 130.805 66.675) (end 130.805 66.375) (width 0.2032) (layer F.Cu) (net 3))
 (segment (start 158.5 76.79) (end 170.46 76.79) (width 0.762) (layer B.Cu) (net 4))
 (segment (start 128.9934 72.25) (end 130 72.25) (width 0.4064) (layer F.Cu) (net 4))
 (segment (start 124.4534 76.79) (end 128.9934 72.25) (width 0.4064) (layer F.Cu) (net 4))
 (segment (start 114.75 76.79) (end 124.4534 76.79) (width 0.4064) (layer F.Cu) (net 4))
 (segment (start 130.805 72.35) (end 130.805 72.05) (width 0.2032) (layer F.Cu) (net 4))
 (segment (start 130 72.25) (end 130.605 72.25) (width 0.3048) (layer F.Cu) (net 4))
 (segment (start 130.605 72.25) (end 130.805 72.05) (width 0.3048) (layer F.Cu) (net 4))
 (segment (start 130 67.25) (end 130.705 67.25) (width 0.3048) (layer F.Cu) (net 4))
 (segment (start 130.705 67.25) (end 130.805 67.15) (width 0.3048) (layer F.Cu) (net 4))
 (segment (start 116.46 76.79) (end 126 67.25) (width 0.4064) (layer F.Cu) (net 4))
 (segment (start 126 67.25) (end 130 67.25) (width 0.4064) (layer F.Cu) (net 4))
 (segment (start 130.805 67.45) (end 130.805 67.15) (width 0.2032) (layer F.Cu) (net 4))
 (segment (start 135.9 65.43) (end 135.9 74.07) (width 0.4064) (layer B.Cu) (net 5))
 (segment (start 135.9 74.07) (end 131.72 74.07) (width 0.4064) (layer B.Cu) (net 5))
 (segment (start 131.72 65.43) (end 135.9 65.43) (width 0.4064) (layer B.Cu) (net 5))
 (segment (start 129.75 70) (end 129.722032 70.027968) (width 0.3048) (layer F.Cu) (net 1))
 (segment (start 130.805 70) (end 129.75 70) (width 0.3048) (layer F.Cu) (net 1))
 (segment (start 129.722032 70.027968) (end 129.671232 70.078768) (width 0.3048) (layer F.Cu) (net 1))
 (segment (start 128.5 71.25) (end 129.671232 70.078768) (width 0.4064) (layer F.Cu) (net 1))
 (segment (start 127.5 71.25) (end 128.5 71.25) (width 0.4064) (layer F.Cu) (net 1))
 (segment (start 129.7752 69.5) (end 130.805 69.5) (width 0.3048) (layer F.Cu) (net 2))
 (segment (start 127.5 69.2) (end 129.45 69.2) (width 0.4064) (layer F.Cu) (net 2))
 (segment (start 129.755241 69.505241) (end 129.45 69.2) (width 0.3048) (layer F.Cu) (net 2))
 (segment (start 129.769959 69.505241) (end 129.7752 69.5) (width 0.3048) (layer F.Cu) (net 2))
 (segment (start 129.769959 69.505241) (end 129.755241 69.505241) (width 0.3048) (layer F.Cu) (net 2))
 (segment (start 129.45 69.2) (end 129.61 69.36) (width 0.4064) (layer F.Cu) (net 2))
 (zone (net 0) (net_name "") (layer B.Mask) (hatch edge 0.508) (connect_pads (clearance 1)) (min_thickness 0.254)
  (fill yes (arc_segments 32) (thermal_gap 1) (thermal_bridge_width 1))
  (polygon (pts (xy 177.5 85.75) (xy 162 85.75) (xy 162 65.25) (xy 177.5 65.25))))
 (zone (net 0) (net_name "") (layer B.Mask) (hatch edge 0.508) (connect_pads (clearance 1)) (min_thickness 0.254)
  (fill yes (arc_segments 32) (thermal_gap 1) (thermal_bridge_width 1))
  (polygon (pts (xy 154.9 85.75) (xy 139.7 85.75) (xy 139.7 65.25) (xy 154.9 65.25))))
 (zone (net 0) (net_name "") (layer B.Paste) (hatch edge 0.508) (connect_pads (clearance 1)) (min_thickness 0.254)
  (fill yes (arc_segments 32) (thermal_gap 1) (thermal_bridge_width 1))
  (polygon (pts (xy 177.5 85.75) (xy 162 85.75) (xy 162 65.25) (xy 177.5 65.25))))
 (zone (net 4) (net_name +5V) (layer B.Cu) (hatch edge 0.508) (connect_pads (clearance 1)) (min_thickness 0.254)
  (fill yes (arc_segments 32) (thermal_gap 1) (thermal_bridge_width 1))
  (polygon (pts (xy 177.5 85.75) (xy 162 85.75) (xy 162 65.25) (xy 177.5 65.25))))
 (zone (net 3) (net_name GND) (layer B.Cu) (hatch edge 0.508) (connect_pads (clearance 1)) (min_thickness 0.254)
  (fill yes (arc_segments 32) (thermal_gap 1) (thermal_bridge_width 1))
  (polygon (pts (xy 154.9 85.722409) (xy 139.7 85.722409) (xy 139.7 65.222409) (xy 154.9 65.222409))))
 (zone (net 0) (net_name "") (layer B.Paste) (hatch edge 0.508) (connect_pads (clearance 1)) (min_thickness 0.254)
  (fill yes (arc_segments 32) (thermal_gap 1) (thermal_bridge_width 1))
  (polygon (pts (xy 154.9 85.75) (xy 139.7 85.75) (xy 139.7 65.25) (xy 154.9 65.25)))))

